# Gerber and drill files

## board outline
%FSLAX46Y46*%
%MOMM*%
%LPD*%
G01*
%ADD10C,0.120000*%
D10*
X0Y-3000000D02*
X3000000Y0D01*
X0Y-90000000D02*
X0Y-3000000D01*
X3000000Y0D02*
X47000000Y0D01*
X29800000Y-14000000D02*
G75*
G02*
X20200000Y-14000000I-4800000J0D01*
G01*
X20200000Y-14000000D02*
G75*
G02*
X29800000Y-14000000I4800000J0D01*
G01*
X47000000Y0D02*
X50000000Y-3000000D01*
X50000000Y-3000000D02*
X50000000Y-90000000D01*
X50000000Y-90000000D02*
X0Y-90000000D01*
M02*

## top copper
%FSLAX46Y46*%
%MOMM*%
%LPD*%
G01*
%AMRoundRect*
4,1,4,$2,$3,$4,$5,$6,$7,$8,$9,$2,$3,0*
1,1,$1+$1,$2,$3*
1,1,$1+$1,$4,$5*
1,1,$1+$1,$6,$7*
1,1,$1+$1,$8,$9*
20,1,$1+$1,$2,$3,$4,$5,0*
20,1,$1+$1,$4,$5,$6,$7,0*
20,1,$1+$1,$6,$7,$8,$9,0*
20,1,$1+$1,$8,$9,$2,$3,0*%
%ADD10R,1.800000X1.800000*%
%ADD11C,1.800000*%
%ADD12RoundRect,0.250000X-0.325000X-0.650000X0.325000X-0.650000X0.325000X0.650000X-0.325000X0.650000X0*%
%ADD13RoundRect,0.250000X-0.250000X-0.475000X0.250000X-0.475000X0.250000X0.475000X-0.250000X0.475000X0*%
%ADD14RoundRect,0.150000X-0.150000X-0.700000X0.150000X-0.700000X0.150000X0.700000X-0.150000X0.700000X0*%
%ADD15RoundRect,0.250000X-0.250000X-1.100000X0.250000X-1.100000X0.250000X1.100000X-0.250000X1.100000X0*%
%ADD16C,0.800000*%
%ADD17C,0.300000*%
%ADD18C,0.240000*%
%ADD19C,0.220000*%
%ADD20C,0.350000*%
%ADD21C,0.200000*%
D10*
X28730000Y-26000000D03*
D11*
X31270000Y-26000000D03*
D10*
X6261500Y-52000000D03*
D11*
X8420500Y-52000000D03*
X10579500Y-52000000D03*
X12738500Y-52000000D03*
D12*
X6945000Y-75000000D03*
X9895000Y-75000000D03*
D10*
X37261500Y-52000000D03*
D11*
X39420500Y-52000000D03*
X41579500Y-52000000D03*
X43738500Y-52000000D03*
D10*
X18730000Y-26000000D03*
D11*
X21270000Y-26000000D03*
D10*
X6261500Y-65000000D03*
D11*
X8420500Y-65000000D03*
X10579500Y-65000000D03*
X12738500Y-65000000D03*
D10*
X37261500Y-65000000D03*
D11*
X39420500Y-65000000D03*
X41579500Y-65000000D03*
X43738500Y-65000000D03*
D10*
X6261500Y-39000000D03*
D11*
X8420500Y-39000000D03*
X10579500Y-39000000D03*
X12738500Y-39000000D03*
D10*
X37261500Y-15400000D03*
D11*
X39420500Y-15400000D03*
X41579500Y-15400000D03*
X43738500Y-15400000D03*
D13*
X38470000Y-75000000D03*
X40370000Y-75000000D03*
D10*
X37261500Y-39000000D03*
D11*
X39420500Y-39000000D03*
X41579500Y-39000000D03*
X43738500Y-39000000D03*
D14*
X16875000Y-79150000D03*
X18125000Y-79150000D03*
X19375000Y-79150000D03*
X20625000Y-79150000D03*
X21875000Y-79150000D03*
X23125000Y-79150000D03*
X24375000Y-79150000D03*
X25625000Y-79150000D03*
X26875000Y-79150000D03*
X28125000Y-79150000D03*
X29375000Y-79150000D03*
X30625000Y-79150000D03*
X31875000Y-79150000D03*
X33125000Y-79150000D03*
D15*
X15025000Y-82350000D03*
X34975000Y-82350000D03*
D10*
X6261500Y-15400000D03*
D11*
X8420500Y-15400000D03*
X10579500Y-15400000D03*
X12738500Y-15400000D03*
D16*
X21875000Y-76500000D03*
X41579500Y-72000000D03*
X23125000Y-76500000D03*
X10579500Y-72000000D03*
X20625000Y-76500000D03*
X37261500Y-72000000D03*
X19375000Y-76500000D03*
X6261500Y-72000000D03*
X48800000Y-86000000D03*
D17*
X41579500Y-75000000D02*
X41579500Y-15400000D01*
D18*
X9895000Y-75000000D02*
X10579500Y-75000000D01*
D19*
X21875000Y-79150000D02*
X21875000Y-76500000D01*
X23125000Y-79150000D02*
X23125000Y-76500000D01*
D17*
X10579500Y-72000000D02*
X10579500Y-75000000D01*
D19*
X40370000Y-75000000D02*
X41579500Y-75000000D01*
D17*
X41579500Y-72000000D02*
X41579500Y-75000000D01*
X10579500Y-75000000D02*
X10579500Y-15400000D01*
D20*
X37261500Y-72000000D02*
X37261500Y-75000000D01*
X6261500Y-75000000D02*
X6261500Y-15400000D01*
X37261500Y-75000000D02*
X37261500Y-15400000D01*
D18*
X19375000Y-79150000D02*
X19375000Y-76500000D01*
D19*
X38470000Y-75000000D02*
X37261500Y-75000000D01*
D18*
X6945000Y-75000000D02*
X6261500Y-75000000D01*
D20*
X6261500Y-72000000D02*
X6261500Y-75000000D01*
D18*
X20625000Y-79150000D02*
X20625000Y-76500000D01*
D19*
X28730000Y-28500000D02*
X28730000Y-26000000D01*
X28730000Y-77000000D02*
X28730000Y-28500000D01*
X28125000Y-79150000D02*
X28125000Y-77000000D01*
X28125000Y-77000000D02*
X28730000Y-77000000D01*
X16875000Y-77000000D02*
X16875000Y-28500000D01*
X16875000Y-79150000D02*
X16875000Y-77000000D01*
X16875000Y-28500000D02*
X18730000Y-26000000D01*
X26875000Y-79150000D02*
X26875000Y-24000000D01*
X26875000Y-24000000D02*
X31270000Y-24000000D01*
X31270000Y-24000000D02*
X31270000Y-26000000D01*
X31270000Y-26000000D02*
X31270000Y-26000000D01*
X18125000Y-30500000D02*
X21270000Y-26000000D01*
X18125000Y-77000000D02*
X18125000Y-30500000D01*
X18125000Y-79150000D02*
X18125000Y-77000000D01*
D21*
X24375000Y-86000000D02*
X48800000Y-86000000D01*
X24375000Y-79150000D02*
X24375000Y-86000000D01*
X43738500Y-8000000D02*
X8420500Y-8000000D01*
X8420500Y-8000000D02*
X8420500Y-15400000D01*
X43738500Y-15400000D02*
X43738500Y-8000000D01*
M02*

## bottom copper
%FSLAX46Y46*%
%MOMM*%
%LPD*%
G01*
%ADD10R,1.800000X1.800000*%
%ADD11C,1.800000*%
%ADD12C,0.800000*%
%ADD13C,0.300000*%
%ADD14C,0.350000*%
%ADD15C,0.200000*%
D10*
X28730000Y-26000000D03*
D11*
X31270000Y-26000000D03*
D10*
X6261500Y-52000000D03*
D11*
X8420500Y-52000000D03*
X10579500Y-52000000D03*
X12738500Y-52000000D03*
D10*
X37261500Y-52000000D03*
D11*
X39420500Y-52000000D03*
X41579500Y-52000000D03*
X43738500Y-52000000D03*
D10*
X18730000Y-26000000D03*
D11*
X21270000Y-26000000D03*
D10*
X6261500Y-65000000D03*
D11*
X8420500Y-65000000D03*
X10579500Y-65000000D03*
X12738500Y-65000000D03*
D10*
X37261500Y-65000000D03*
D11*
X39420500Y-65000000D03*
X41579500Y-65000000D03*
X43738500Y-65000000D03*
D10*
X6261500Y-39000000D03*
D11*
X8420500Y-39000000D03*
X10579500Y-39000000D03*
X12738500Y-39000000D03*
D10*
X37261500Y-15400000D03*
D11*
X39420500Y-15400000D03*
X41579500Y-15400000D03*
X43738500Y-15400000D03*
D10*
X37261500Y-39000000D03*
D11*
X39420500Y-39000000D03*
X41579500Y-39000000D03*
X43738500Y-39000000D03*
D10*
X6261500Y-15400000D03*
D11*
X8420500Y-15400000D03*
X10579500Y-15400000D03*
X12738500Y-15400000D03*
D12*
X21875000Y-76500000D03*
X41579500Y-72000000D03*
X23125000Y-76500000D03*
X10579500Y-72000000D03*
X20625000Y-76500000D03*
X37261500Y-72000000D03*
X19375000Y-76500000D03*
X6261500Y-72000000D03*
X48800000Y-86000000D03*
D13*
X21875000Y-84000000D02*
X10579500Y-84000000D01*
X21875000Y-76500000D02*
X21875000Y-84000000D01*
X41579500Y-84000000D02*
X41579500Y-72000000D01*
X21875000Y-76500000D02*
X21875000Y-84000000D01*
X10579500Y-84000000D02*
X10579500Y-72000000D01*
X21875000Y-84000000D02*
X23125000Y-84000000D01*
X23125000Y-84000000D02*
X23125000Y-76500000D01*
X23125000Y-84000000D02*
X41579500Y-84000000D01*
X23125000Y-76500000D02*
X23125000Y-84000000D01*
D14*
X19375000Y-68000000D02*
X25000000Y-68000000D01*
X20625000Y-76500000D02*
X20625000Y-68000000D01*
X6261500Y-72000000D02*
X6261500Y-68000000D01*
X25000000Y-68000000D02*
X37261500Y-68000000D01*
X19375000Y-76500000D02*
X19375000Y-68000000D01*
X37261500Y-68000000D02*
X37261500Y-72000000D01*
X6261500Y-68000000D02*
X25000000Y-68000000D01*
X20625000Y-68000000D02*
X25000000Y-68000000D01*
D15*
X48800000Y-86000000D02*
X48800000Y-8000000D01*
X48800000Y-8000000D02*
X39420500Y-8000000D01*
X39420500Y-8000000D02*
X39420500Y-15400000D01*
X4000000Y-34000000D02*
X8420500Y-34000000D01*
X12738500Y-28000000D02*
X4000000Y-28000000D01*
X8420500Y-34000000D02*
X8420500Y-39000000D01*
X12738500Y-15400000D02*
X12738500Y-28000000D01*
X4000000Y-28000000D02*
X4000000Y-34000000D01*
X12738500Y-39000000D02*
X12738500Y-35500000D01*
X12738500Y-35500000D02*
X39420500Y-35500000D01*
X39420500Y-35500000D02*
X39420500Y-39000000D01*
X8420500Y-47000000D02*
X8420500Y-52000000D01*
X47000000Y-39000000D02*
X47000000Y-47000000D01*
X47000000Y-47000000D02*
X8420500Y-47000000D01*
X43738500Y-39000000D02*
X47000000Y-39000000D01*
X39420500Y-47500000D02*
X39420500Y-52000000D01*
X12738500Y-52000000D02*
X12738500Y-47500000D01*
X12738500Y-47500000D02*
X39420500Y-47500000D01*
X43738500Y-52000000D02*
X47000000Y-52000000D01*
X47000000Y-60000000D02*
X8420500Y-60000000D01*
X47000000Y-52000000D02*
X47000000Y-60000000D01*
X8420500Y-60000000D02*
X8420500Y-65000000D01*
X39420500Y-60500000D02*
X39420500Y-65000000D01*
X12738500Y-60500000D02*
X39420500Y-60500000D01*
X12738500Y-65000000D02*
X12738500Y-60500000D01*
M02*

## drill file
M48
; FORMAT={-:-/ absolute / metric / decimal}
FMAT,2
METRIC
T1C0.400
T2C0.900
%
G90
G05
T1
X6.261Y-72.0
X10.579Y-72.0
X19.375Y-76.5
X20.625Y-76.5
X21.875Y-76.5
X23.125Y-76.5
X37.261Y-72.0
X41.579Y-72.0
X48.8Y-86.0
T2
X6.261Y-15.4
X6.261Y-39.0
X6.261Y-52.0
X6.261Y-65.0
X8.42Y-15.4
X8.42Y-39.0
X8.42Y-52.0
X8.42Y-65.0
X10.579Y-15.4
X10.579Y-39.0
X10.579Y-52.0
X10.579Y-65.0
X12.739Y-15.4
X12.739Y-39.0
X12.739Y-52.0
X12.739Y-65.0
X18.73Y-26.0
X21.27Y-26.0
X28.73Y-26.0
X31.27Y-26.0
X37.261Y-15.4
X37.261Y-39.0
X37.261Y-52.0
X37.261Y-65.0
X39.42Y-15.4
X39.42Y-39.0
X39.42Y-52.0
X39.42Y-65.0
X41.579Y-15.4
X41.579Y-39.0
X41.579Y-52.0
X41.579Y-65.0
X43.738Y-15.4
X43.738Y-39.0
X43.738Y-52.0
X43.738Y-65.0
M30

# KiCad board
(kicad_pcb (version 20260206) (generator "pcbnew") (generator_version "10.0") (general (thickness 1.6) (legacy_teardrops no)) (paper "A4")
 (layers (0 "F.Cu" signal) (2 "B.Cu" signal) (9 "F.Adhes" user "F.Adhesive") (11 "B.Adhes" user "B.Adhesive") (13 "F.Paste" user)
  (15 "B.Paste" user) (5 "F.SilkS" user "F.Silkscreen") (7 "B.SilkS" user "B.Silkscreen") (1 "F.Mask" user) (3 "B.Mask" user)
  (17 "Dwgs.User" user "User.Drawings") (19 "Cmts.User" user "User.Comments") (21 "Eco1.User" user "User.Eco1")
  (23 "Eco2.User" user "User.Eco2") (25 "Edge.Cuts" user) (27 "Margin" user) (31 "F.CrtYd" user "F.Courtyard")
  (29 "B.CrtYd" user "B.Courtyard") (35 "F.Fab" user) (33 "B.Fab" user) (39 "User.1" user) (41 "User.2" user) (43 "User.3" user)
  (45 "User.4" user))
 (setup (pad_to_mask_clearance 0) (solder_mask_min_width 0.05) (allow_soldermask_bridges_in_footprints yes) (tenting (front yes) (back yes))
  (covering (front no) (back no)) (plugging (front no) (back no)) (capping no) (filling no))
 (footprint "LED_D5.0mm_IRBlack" (layer "F.Cu") (at 28.73 26)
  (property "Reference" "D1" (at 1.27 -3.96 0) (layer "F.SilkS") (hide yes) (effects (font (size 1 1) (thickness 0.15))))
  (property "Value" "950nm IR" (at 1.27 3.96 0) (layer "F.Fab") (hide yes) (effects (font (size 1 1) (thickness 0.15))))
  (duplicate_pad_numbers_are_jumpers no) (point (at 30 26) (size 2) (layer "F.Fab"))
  (pad "1" thru_hole rect (at 0 0) (size 1.8 1.8) (drill 0.9) (layers "*.Cu" "*.Mask") (remove_unused_layers no) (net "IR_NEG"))
  (pad "2" thru_hole circle (at 2.54 0) (size 1.8 1.8) (drill 0.9) (layers "*.Cu" "*.Mask") (remove_unused_layers no) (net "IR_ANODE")))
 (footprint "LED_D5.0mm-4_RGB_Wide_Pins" (layer "F.Cu") (at 6.2615 52)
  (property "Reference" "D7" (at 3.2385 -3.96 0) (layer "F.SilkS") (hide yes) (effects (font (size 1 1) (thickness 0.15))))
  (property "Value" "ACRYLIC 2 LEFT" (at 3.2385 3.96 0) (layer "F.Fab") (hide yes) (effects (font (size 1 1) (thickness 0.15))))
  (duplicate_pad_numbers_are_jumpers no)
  (pad "1" thru_hole rect (at 0 0) (size 1.8 1.8) (drill 0.9) (layers "*.Cu" "*.Mask") (remove_unused_layers no) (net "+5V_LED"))
  (pad "2" thru_hole circle (at 2.159 0) (size 1.8 1.8) (drill 0.9) (layers "*.Cu" "*.Mask") (remove_unused_layers no) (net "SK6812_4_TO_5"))
  (pad "3" thru_hole circle (at 4.318 0) (size 1.8 1.8) (drill 0.9) (layers "*.Cu" "*.Mask") (remove_unused_layers no) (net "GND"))
  (pad "4" thru_hole circle (at 6.477 0) (size 1.8 1.8) (drill 0.9) (layers "*.Cu" "*.Mask") (remove_unused_layers no) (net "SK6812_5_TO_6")))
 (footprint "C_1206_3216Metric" (layer "F.Cu") (at 8.42 75)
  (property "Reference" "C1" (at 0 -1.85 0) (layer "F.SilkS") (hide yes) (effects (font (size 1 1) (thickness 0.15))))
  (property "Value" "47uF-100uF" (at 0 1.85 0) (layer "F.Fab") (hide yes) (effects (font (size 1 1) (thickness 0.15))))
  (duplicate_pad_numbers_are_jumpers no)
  (pad "1" smd roundrect (at -1.475 0) (size 1.15 1.8) (layers "F.Cu" "F.Mask" "F.Paste") (roundrect_rratio 0.217391) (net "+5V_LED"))
  (pad "2" smd roundrect (at 1.475 0) (size 1.15 1.8) (layers "F.Cu" "F.Mask" "F.Paste") (roundrect_rratio 0.217391) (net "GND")))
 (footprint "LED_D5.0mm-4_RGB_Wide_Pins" (layer "F.Cu") (at 37.2615 52)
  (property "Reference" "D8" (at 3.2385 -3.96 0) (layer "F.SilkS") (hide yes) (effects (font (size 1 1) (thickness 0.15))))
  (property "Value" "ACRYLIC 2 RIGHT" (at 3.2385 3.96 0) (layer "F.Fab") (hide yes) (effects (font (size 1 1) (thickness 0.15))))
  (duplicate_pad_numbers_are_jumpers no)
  (pad "1" thru_hole rect (at 0 0) (size 1.8 1.8) (drill 0.9) (layers "*.Cu" "*.Mask") (remove_unused_layers no) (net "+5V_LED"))
  (pad "2" thru_hole circle (at 2.159 0) (size 1.8 1.8) (drill 0.9) (layers "*.Cu" "*.Mask") (remove_unused_layers no) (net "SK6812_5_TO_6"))
  (pad "3" thru_hole circle (at 4.318 0) (size 1.8 1.8) (drill 0.9) (layers "*.Cu" "*.Mask") (remove_unused_layers no) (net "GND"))
  (pad "4" thru_hole circle (at 6.477 0) (size 1.8 1.8) (drill 0.9) (layers "*.Cu" "*.Mask") (remove_unused_layers no) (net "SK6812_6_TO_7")))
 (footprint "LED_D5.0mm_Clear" (layer "F.Cu") (at 18.73 26)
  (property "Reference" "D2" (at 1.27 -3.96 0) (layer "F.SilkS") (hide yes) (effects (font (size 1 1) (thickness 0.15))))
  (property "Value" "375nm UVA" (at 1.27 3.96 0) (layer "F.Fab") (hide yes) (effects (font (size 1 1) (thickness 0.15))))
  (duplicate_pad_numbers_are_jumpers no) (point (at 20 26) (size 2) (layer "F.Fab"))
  (pad "1" thru_hole rect (at 0 0) (size 1.8 1.8) (drill 0.9) (layers "*.Cu" "*.Mask") (remove_unused_layers no) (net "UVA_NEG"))
  (pad "2" thru_hole circle (at 2.54 0) (size 1.8 1.8) (drill 0.9) (layers "*.Cu" "*.Mask") (remove_unused_layers no) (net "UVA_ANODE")))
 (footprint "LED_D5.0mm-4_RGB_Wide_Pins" (layer "F.Cu") (at 6.2615 65)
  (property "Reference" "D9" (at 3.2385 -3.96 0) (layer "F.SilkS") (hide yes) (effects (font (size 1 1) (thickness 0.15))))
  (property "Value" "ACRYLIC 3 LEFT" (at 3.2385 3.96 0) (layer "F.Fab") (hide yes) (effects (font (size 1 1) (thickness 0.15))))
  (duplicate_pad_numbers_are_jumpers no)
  (pad "1" thru_hole rect (at 0 0) (size 1.8 1.8) (drill 0.9) (layers "*.Cu" "*.Mask") (remove_unused_layers no) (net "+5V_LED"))
  (pad "2" thru_hole circle (at 2.159 0) (size 1.8 1.8) (drill 0.9) (layers "*.Cu" "*.Mask") (remove_unused_layers no) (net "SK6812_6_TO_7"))
  (pad "3" thru_hole circle (at 4.318 0) (size 1.8 1.8) (drill 0.9) (layers "*.Cu" "*.Mask") (remove_unused_layers no) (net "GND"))
  (pad "4" thru_hole circle (at 6.477 0) (size 1.8 1.8) (drill 0.9) (layers "*.Cu" "*.Mask") (remove_unused_layers no) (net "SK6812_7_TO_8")))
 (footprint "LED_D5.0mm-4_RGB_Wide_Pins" (layer "F.Cu") (at 37.2615 65)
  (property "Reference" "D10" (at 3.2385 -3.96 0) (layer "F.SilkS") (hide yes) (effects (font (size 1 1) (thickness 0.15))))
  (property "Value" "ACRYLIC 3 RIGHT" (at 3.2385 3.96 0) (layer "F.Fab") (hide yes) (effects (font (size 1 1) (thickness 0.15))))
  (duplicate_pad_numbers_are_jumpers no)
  (pad "1" thru_hole rect (at 0 0) (size 1.8 1.8) (drill 0.9) (layers "*.Cu" "*.Mask") (remove_unused_layers no) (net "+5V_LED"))
  (pad "2" thru_hole circle (at 2.159 0) (size 1.8 1.8) (drill 0.9) (layers "*.Cu" "*.Mask") (remove_unused_layers no) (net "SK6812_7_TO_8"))
  (pad "3" thru_hole circle (at 4.318 0) (size 1.8 1.8) (drill 0.9) (layers "*.Cu" "*.Mask") (remove_unused_layers no) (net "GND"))
  (pad "4" thru_hole circle (at 6.477 0) (size 1.8 1.8) (drill 0.9) (layers "*.Cu" "*.Mask") (remove_unused_layers no)))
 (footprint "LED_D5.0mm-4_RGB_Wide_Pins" (layer "F.Cu") (at 6.2615 39)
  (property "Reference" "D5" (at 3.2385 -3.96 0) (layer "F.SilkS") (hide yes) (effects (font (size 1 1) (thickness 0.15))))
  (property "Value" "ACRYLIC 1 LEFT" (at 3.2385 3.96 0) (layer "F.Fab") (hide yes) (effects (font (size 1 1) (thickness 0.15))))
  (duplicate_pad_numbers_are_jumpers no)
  (pad "1" thru_hole rect (at 0 0) (size 1.8 1.8) (drill 0.9) (layers "*.Cu" "*.Mask") (remove_unused_layers no) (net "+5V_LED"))
  (pad "2" thru_hole circle (at 2.159 0) (size 1.8 1.8) (drill 0.9) (layers "*.Cu" "*.Mask") (remove_unused_layers no) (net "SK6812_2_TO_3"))
  (pad "3" thru_hole circle (at 4.318 0) (size 1.8 1.8) (drill 0.9) (layers "*.Cu" "*.Mask") (remove_unused_layers no) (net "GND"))
  (pad "4" thru_hole circle (at 6.477 0) (size 1.8 1.8) (drill 0.9) (layers "*.Cu" "*.Mask") (remove_unused_layers no) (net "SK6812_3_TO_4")))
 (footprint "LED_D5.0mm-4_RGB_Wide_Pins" (layer "F.Cu") (at 37.2615 15.4)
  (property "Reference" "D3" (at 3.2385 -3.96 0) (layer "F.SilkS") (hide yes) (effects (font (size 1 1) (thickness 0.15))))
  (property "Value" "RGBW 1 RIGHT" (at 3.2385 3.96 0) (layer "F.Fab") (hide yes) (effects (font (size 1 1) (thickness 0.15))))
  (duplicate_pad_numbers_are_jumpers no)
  (pad "1" thru_hole rect (at 0 0) (size 1.8 1.8) (drill 0.9) (layers "*.Cu" "*.Mask") (remove_unused_layers no) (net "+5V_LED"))
  (pad "2" thru_hole circle (at 2.159 0) (size 1.8 1.8) (drill 0.9) (layers "*.Cu" "*.Mask") (remove_unused_layers no) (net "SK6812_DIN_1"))
  (pad "3" thru_hole circle (at 4.318 0) (size 1.8 1.8) (drill 0.9) (layers "*.Cu" "*.Mask") (remove_unused_layers no) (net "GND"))
  (pad "4" thru_hole circle (at 6.477 0) (size 1.8 1.8) (drill 0.9) (layers "*.Cu" "*.Mask") (remove_unused_layers no) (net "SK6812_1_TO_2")))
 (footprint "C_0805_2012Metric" (layer "F.Cu") (at 39.42 75)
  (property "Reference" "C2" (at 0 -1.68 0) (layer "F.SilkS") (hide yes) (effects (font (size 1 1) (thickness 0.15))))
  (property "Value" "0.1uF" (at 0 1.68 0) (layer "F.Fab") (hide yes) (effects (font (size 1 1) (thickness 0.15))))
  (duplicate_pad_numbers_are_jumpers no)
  (pad "1" smd roundrect (at -0.95 0) (size 1 1.45) (layers "F.Cu" "F.Mask" "F.Paste") (roundrect_rratio 0.25) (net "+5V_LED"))
  (pad "2" smd roundrect (at 0.95 0) (size 1 1.45) (layers "F.Cu" "F.Mask" "F.Paste") (roundrect_rratio 0.25) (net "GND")))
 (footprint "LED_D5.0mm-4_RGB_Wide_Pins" (layer "F.Cu") (at 37.2615 39)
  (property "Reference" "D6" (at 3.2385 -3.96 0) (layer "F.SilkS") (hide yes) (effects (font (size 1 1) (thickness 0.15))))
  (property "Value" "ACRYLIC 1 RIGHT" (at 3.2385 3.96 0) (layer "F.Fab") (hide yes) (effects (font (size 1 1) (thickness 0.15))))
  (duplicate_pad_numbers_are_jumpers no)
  (pad "1" thru_hole rect (at 0 0) (size 1.8 1.8) (drill 0.9) (layers "*.Cu" "*.Mask") (remove_unused_layers no) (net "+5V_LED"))
  (pad "2" thru_hole circle (at 2.159 0) (size 1.8 1.8) (drill 0.9) (layers "*.Cu" "*.Mask") (remove_unused_layers no) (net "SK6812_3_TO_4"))
  (pad "3" thru_hole circle (at 4.318 0) (size 1.8 1.8) (drill 0.9) (layers "*.Cu" "*.Mask") (remove_unused_layers no) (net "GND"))
  (pad "4" thru_hole circle (at 6.477 0) (size 1.8 1.8) (drill 0.9) (layers "*.Cu" "*.Mask") (remove_unused_layers no) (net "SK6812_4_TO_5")))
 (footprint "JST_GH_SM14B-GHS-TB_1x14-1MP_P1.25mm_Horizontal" (layer "F.Cu") (at 25 81)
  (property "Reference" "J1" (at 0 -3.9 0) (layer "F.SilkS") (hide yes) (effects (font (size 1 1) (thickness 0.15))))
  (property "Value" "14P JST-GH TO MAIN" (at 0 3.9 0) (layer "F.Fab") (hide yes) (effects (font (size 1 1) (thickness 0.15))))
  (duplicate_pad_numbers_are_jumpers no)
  (pad "1" smd roundrect (at -8.125 -1.85) (size 0.6 1.7) (layers "F.Cu" "F.Mask" "F.Paste") (roundrect_rratio 0.25) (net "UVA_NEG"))
  (pad "2" smd roundrect (at -6.875 -1.85) (size 0.6 1.7) (layers "F.Cu" "F.Mask" "F.Paste") (roundrect_rratio 0.25) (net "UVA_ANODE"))
  (pad "3" smd roundrect (at -5.625 -1.85) (size 0.6 1.7) (layers "F.Cu" "F.Mask" "F.Paste") (roundrect_rratio 0.25) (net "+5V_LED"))
  (pad "4" smd roundrect (at -4.375 -1.85) (size 0.6 1.7) (layers "F.Cu" "F.Mask" "F.Paste") (roundrect_rratio 0.25) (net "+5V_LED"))
  (pad "5" smd roundrect (at -3.125 -1.85) (size 0.6 1.7) (layers "F.Cu" "F.Mask" "F.Paste") (roundrect_rratio 0.25) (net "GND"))
  (pad "6" smd roundrect (at -1.875 -1.85) (size 0.6 1.7) (layers "F.Cu" "F.Mask" "F.Paste") (roundrect_rratio 0.25) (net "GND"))
  (pad "7" smd roundrect (at -0.625 -1.85) (size 0.6 1.7) (layers "F.Cu" "F.Mask" "F.Paste") (roundrect_rratio 0.25) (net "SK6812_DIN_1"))
  (pad "8" smd roundrect (at 0.625 -1.85) (size 0.6 1.7) (layers "F.Cu" "F.Mask" "F.Paste") (roundrect_rratio 0.25))
  (pad "9" smd roundrect (at 1.875 -1.85) (size 0.6 1.7) (layers "F.Cu" "F.Mask" "F.Paste") (roundrect_rratio 0.25) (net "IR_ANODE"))
  (pad "10" smd roundrect (at 3.125 -1.85) (size 0.6 1.7) (layers "F.Cu" "F.Mask" "F.Paste") (roundrect_rratio 0.25) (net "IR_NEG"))
  (pad "11" smd roundrect (at 4.375 -1.85) (size 0.6 1.7) (layers "F.Cu" "F.Mask" "F.Paste") (roundrect_rratio 0.25))
  (pad "12" smd roundrect (at 5.625 -1.85) (size 0.6 1.7) (layers "F.Cu" "F.Mask" "F.Paste") (roundrect_rratio 0.25))
  (pad "13" smd roundrect (at 6.875 -1.85) (size 0.6 1.7) (layers "F.Cu" "F.Mask" "F.Paste") (roundrect_rratio 0.25))
  (pad "14" smd roundrect (at 8.125 -1.85) (size 0.6 1.7) (layers "F.Cu" "F.Mask" "F.Paste") (roundrect_rratio 0.25))
  (pad "MP" smd roundrect (at -9.975 1.35) (size 1 2.7) (layers "F.Cu" "F.Mask" "F.Paste") (roundrect_rratio 0.25))
  (pad "MP" smd roundrect (at 9.975 1.35) (size 1 2.7) (layers "F.Cu" "F.Mask" "F.Paste") (roundrect_rratio 0.25)))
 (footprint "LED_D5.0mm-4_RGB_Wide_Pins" (layer "F.Cu") (at 6.2615 15.4)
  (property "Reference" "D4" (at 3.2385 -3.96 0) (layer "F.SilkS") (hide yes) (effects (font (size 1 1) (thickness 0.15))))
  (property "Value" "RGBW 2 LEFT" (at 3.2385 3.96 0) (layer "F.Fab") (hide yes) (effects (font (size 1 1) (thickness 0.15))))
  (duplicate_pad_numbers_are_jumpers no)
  (pad "1" thru_hole rect (at 0 0) (size 1.8 1.8) (drill 0.9) (layers "*.Cu" "*.Mask") (remove_unused_layers no) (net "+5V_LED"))
  (pad "2" thru_hole circle (at 2.159 0) (size 1.8 1.8) (drill 0.9) (layers "*.Cu" "*.Mask") (remove_unused_layers no) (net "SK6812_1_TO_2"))
  (pad "3" thru_hole circle (at 4.318 0) (size 1.8 1.8) (drill 0.9) (layers "*.Cu" "*.Mask") (remove_unused_layers no) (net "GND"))
  (pad "4" thru_hole circle (at 6.477 0) (size 1.8 1.8) (drill 0.9) (layers "*.Cu" "*.Mask") (remove_unused_layers no) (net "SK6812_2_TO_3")))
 (gr_line (start 0 3) (end 3 0) (stroke (width 0.12) (type default)) (layer "Edge.Cuts"))
 (gr_line (start 0 90) (end 0 3) (stroke (width 0.12) (type default)) (layer "Edge.Cuts"))
 (gr_line (start 3 0) (end 47 0) (stroke (width 0.12) (type default)) (layer "Edge.Cuts"))
 (gr_circle (center 25 14) (end 29.8 14) (stroke (width 0.12) (type default)) (fill no) (layer "Edge.Cuts"))
 (gr_line (start 47 0) (end 50 3) (stroke (width 0.12) (type default)) (layer "Edge.Cuts"))
 (gr_line (start 50 3) (end 50 90) (stroke (width 0.12) (type default)) (layer "Edge.Cuts"))
 (gr_line (start 50 90) (end 0 90) (stroke (width 0.12) (type default)) (layer "Edge.Cuts"))
 (segment (start 41.5795 75) (end 41.5795 15.4) (width 0.3) (layer "F.Cu") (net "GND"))
 (segment (start 9.895 75) (end 10.5795 75) (width 0.24) (layer "F.Cu") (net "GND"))
 (segment (start 21.875 79.15) (end 21.875 76.5) (width 0.22) (layer "F.Cu") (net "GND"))
 (segment (start 23.125 79.15) (end 23.125 76.5) (width 0.22) (layer "F.Cu") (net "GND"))
 (segment (start 10.5795 72) (end 10.5795 75) (width 0.3) (layer "F.Cu") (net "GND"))
 (segment (start 40.37 75) (end 41.5795 75) (width 0.22) (layer "F.Cu") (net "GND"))
 (segment (start 41.5795 72) (end 41.5795 75) (width 0.3) (layer "F.Cu") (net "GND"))
 (segment (start 10.5795 75) (end 10.5795 15.4) (width 0.3) (layer "F.Cu") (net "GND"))
 (via (at 21.875 76.5) (size 0.8) (drill 0.4) (layers "F.Cu" "B.Cu") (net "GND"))
 (via (at 41.5795 72) (size 0.8) (drill 0.4) (layers "F.Cu" "B.Cu") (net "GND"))
 (via (at 23.125 76.5) (size 0.8) (drill 0.4) (layers "F.Cu" "B.Cu") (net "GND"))
 (via (at 10.5795 72) (size 0.8) (drill 0.4) (layers "F.Cu" "B.Cu") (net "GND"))
 (segment (start 21.875 84) (end 10.5795 84) (width 0.3) (layer "B.Cu") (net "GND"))
 (segment (start 21.875 76.5) (end 21.875 84) (width 0.3) (layer "B.Cu") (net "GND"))
 (segment (start 41.5795 84) (end 41.5795 72) (width 0.3) (layer "B.Cu") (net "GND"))
 (segment (start 21.875 76.5) (end 21.875 84) (width 0.3) (layer "B.Cu") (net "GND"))
 (segment (start 10.5795 84) (end 10.5795 72) (width 0.3) (layer "B.Cu") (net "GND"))
 (segment (start 21.875 84) (end 23.125 84) (width 0.3) (layer "B.Cu") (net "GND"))
 (segment (start 23.125 84) (end 23.125 76.5) (width 0.3) (layer "B.Cu") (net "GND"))
 (segment (start 23.125 84) (end 41.5795 84) (width 0.3) (layer "B.Cu") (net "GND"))
 (segment (start 23.125 76.5) (end 23.125 84) (width 0.3) (layer "B.Cu") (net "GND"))
 (segment (start 37.2615 72) (end 37.2615 75) (width 0.35) (layer "F.Cu") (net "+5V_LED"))
 (segment (start 6.2615 75) (end 6.2615 15.4) (width 0.35) (layer "F.Cu") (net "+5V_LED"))
 (segment (start 37.2615 75) (end 37.2615 15.4) (width 0.35) (layer "F.Cu") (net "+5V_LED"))
 (segment (start 19.375 79.15) (end 19.375 76.5) (width 0.24) (layer "F.Cu") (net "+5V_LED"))
 (segment (start 38.47 75) (end 37.2615 75) (width 0.22) (layer "F.Cu") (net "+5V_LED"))
 (segment (start 6.945 75) (end 6.2615 75) (width 0.24) (layer "F.Cu") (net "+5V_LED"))
 (segment (start 6.2615 72) (end 6.2615 75) (width 0.35) (layer "F.Cu") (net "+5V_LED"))
 (segment (start 20.625 79.15) (end 20.625 76.5) (width 0.24) (layer "F.Cu") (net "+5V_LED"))
 (via (at 20.625 76.5) (size 0.8) (drill 0.4) (layers "F.Cu" "B.Cu") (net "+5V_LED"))
 (via (at 37.2615 72) (size 0.8) (drill 0.4) (layers "F.Cu" "B.Cu") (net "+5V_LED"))
 (via (at 19.375 76.5) (size 0.8) (drill 0.4) (layers "F.Cu" "B.Cu") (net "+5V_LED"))
 (via (at 6.2615 72) (size 0.8) (drill 0.4) (layers "F.Cu" "B.Cu") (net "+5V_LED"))
 (segment (start 19.375 68) (end 25 68) (width 0.35) (layer "B.Cu") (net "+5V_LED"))
 (segment (start 20.625 76.5) (end 20.625 68) (width 0.35) (layer "B.Cu") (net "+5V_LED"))
 (segment (start 6.2615 72) (end 6.2615 68) (width 0.35) (layer "B.Cu") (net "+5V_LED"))
 (segment (start 25 68) (end 37.2615 68) (width 0.35) (layer "B.Cu") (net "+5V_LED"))
 (segment (start 19.375 76.5) (end 19.375 68) (width 0.35) (layer "B.Cu") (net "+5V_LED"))
 (segment (start 37.2615 68) (end 37.2615 72) (width 0.35) (layer "B.Cu") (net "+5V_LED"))
 (segment (start 6.2615 68) (end 25 68) (width 0.35) (layer "B.Cu") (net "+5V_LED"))
 (segment (start 20.625 68) (end 25 68) (width 0.35) (layer "B.Cu") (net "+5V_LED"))
 (segment (start 28.73 28.5) (end 28.73 26) (width 0.22) (layer "F.Cu") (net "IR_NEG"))
 (segment (start 28.73 77) (end 28.73 28.5) (width 0.22) (layer "F.Cu") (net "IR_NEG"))
 (segment (start 28.125 79.15) (end 28.125 77) (width 0.22) (layer "F.Cu") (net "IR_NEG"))
 (segment (start 28.125 77) (end 28.73 77) (width 0.22) (layer "F.Cu") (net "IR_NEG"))
 (segment (start 16.875 77) (end 16.875 28.5) (width 0.22) (layer "F.Cu") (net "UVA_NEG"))
 (segment (start 16.875 79.15) (end 16.875 77) (width 0.22) (layer "F.Cu") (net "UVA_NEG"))
 (segment (start 16.875 28.5) (end 18.73 26) (width 0.22) (layer "F.Cu") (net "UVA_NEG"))
 (segment (start 26.875 79.15) (end 26.875 24) (width 0.22) (layer "F.Cu") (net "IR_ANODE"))
 (segment (start 26.875 24) (end 31.27 24) (width 0.22) (layer "F.Cu") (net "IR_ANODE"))
 (segment (start 31.27 24) (end 31.27 26) (width 0.22) (layer "F.Cu") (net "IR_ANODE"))
 (segment (start 31.27 26) (end 31.27 26) (width 0.22) (layer "F.Cu") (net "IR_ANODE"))
 (segment (start 18.125 30.5) (end 21.27 26) (width 0.22) (layer "F.Cu") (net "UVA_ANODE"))
 (segment (start 18.125 77) (end 18.125 30.5) (width 0.22) (layer "F.Cu") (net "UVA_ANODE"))
 (segment (start 18.125 79.15) (end 18.125 77) (width 0.22) (layer "F.Cu") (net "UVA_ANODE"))
 (segment (start 24.375 86) (end 48.8 86) (width 0.2) (layer "F.Cu") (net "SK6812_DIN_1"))
 (segment (start 24.375 79.15) (end 24.375 86) (width 0.2) (layer "F.Cu") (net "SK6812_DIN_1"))
 (via (at 48.8 86) (size 0.8) (drill 0.4) (layers "F.Cu" "B.Cu") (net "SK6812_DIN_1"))
 (segment (start 48.8 86) (end 48.8 8) (width 0.2) (layer "B.Cu") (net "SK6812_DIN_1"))
 (segment (start 48.8 8) (end 39.4205 8) (width 0.2) (layer "B.Cu") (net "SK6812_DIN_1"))
 (segment (start 39.4205 8) (end 39.4205 15.4) (width 0.2) (layer "B.Cu") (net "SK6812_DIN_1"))
 (segment (start 43.7385 8) (end 8.4205 8) (width 0.2) (layer "F.Cu") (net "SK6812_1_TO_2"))
 (segment (start 8.4205 8) (end 8.4205 15.4) (width 0.2) (layer "F.Cu") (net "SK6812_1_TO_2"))
 (segment (start 43.7385 15.4) (end 43.7385 8) (width 0.2) (layer "F.Cu") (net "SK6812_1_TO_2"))
 (segment (start 4 34) (end 8.4205 34) (width 0.2) (layer "B.Cu") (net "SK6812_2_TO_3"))
 (segment (start 12.7385 28) (end 4 28) (width 0.2) (layer "B.Cu") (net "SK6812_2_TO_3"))
 (segment (start 8.4205 34) (end 8.4205 39) (width 0.2) (layer "B.Cu") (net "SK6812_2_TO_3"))
 (segment (start 12.7385 15.4) (end 12.7385 28) (width 0.2) (layer "B.Cu") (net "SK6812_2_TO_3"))
 (segment (start 4 28) (end 4 34) (width 0.2) (layer "B.Cu") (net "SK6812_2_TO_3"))
 (segment (start 12.7385 39) (end 12.7385 35.5) (width 0.2) (layer "B.Cu") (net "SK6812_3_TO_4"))
 (segment (start 12.7385 35.5) (end 39.4205 35.5) (width 0.2) (layer "B.Cu") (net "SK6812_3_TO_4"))
 (segment (start 39.4205 35.5) (end 39.4205 39) (width 0.2) (layer "B.Cu") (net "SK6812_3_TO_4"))
 (segment (start 8.4205 47) (end 8.4205 52) (width 0.2) (layer "B.Cu") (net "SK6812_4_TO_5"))
 (segment (start 47 39) (end 47 47) (width 0.2) (layer "B.Cu") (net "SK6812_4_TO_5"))
 (segment (start 47 47) (end 8.4205 47) (width 0.2) (layer "B.Cu") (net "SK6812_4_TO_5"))
 (segment (start 43.7385 39) (end 47 39) (width 0.2) (layer "B.Cu") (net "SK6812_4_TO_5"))
 (segment (start 39.4205 47.5) (end 39.4205 52) (width 0.2) (layer "B.Cu") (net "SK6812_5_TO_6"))
 (segment (start 12.7385 52) (end 12.7385 47.5) (width 0.2) (layer "B.Cu") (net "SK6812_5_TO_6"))
 (segment (start 12.7385 47.5) (end 39.4205 47.5) (width 0.2) (layer "B.Cu") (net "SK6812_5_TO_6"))
 (segment (start 43.7385 52) (end 47 52) (width 0.2) (layer "B.Cu") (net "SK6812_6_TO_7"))
 (segment (start 47 60) (end 8.4205 60) (width 0.2) (layer "B.Cu") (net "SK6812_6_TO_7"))
 (segment (start 47 52) (end 47 60) (width 0.2) (layer "B.Cu") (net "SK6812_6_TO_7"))
 (segment (start 8.4205 60) (end 8.4205 65) (width 0.2) (layer "B.Cu") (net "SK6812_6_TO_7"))
 (segment (start 39.4205 60.5) (end 39.4205 65) (width 0.2) (layer "B.Cu") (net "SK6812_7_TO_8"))
 (segment (start 12.7385 60.5) (end 39.4205 60.5) (width 0.2) (layer "B.Cu") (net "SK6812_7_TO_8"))
 (segment (start 12.7385 65) (end 12.7385 60.5) (width 0.2) (layer "B.Cu") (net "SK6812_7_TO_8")))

